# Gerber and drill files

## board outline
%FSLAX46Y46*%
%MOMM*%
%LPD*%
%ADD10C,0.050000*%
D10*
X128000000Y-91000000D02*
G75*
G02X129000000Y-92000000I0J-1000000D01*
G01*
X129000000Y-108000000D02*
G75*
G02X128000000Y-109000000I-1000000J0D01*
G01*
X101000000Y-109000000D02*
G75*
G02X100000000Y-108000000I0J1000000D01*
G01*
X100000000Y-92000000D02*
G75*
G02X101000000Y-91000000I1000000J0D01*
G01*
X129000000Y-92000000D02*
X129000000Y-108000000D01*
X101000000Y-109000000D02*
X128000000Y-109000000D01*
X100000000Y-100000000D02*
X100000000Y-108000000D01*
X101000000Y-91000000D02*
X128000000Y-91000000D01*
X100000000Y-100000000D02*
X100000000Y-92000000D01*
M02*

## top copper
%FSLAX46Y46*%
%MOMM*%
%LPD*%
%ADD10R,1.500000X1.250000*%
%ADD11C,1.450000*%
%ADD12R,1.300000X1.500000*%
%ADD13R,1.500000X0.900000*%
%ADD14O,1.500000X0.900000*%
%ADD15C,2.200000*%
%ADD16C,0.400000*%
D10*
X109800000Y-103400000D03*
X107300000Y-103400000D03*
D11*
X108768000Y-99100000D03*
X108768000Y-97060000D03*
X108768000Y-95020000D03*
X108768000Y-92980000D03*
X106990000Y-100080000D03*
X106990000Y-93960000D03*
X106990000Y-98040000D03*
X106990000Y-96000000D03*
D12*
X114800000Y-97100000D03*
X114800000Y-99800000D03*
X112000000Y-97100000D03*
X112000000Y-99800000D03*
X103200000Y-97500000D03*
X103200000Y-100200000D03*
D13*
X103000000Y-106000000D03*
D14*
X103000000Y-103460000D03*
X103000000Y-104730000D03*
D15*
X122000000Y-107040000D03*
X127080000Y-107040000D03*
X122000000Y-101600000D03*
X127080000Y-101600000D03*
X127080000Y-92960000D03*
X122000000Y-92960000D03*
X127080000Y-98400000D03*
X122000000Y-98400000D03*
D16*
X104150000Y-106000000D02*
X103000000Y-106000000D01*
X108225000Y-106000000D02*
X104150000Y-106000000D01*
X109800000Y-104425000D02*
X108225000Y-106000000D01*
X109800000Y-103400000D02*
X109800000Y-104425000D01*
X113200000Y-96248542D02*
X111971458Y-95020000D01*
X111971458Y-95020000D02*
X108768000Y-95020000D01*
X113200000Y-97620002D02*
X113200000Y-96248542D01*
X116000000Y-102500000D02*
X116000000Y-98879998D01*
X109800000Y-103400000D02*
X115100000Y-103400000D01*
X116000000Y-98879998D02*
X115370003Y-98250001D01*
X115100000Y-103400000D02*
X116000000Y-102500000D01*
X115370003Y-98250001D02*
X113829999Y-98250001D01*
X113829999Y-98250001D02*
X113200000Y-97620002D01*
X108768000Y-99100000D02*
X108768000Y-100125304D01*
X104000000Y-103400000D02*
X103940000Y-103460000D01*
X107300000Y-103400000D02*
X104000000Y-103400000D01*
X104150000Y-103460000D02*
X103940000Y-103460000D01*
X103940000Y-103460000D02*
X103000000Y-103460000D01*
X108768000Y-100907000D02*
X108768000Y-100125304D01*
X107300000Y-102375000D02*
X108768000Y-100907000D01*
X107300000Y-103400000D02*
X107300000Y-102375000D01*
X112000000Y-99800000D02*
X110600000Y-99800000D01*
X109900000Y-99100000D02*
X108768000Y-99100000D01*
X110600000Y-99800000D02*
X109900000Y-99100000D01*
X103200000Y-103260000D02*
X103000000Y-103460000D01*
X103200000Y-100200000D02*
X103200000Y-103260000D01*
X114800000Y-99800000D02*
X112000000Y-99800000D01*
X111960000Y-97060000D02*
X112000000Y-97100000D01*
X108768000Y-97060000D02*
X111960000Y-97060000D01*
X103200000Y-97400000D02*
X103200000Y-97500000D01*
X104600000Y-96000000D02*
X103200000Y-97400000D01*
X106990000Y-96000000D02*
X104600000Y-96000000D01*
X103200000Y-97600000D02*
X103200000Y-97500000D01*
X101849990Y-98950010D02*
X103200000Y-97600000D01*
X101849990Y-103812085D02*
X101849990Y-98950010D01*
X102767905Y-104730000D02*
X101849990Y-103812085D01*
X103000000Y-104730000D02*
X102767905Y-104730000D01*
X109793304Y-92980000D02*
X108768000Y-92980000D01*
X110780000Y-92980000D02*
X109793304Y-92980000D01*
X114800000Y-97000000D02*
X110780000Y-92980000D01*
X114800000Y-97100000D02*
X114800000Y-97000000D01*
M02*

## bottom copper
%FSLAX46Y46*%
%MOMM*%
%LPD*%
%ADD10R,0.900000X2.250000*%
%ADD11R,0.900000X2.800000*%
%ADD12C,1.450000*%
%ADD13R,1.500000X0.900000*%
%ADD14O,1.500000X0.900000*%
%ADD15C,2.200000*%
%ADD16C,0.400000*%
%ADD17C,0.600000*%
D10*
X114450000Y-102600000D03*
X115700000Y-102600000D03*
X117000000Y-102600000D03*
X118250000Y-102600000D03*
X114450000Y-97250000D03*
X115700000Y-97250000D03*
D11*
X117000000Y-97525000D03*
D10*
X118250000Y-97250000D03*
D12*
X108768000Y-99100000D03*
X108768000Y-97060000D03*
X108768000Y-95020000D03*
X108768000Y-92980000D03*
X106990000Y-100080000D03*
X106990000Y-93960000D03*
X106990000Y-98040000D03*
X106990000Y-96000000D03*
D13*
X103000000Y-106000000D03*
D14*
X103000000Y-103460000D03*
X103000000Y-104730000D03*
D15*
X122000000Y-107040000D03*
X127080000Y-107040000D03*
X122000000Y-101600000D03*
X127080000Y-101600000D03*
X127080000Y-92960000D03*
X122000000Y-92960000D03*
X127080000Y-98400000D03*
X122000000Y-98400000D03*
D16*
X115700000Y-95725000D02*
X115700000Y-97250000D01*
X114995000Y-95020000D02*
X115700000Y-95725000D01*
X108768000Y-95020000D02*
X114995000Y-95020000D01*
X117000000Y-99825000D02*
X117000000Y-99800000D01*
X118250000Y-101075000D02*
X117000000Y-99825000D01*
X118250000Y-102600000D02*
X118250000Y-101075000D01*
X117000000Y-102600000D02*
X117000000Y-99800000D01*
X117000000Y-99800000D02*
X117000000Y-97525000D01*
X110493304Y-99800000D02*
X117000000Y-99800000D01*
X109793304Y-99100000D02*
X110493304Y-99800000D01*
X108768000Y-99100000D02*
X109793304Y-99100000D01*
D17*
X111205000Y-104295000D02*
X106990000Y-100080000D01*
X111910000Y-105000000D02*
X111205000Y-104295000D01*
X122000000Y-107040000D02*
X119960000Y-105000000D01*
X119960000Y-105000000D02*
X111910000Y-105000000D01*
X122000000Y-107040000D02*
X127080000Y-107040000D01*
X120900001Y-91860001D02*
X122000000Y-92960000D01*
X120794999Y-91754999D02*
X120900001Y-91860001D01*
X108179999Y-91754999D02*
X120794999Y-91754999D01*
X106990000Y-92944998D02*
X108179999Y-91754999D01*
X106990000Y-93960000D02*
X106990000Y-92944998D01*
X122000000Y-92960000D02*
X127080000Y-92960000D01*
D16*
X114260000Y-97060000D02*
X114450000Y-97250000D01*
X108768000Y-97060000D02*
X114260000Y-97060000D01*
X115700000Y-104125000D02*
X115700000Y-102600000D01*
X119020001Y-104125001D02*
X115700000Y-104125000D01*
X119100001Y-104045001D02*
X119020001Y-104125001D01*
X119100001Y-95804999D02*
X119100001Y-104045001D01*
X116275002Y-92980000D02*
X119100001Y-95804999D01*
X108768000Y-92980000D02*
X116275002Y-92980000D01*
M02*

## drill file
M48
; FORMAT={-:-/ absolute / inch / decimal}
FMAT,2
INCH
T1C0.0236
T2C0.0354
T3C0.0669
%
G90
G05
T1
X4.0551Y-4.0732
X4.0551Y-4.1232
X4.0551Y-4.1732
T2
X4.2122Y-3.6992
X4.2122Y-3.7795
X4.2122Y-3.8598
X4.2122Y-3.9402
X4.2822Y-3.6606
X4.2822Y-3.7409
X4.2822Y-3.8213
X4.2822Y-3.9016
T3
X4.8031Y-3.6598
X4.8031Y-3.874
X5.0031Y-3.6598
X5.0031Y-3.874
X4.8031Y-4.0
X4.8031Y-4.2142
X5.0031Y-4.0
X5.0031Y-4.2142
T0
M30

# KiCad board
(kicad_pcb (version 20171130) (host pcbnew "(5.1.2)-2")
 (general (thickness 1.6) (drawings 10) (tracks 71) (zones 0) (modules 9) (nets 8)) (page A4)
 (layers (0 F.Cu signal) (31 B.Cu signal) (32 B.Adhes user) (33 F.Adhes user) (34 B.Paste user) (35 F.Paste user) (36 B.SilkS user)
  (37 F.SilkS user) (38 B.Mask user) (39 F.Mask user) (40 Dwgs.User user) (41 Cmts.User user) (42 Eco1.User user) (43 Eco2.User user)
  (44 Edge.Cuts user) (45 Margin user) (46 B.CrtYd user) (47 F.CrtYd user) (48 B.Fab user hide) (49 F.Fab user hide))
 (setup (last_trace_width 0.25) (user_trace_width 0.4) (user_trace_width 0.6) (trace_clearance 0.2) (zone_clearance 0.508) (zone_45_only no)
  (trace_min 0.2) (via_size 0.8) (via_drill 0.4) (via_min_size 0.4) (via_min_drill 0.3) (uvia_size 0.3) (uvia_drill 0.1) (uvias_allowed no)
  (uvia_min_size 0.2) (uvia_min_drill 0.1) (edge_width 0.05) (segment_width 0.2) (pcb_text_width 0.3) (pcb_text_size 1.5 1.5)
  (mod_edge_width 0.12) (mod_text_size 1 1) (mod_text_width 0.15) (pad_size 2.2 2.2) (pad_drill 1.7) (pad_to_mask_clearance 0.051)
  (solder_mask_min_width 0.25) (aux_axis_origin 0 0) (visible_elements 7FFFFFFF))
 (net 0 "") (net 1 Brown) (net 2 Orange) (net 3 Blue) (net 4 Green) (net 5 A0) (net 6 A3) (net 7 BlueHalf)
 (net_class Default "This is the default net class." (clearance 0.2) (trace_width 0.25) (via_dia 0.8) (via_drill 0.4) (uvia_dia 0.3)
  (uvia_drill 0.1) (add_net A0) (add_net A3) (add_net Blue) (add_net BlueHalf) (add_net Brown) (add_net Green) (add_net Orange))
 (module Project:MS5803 (layer B.Cu) (at 116.35 100 90)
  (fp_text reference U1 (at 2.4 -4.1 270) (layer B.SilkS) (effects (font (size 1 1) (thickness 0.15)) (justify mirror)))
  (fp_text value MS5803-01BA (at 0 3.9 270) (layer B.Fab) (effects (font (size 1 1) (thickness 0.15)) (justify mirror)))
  (pad 8 smd rect (at -2.6 -1.9 90) (size 2.25 0.9) (layers B.Cu B.Paste B.Mask) (solder_mask_margin 0.1))
  (pad 7 smd rect (at -2.6 -0.65 90) (size 2.25 0.9) (layers B.Cu B.Paste B.Mask) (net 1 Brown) (solder_mask_margin 0.1))
  (pad 6 smd rect (at -2.6 0.65 90) (size 2.25 0.9) (layers B.Cu B.Paste B.Mask) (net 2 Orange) (solder_mask_margin 0.1))
  (pad 5 smd rect (at -2.6 1.9 90) (size 2.25 0.9) (layers B.Cu B.Paste B.Mask) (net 2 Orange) (solder_mask_margin 0.1))
  (pad 1 smd rect (at 2.75 -1.9 90) (size 2.25 0.9) (layers B.Cu B.Paste B.Mask) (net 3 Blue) (solder_mask_margin 0.1))
  (pad 2 smd rect (at 2.75 -0.65 90) (size 2.25 0.9) (layers B.Cu B.Paste B.Mask) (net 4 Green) (solder_mask_margin 0.1))
  (pad 3 smd rect (at 2.475 0.65 90) (size 2.8 0.9) (layers B.Cu B.Paste B.Mask) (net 2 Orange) (solder_mask_margin 0.1))
  (pad 4 smd rect (at 2.75 1.9 90) (size 2.25 0.9) (layers B.Cu B.Paste B.Mask) (solder_mask_margin 0.1)))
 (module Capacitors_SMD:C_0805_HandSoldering (layer F.Cu) (at 108.55 103.4)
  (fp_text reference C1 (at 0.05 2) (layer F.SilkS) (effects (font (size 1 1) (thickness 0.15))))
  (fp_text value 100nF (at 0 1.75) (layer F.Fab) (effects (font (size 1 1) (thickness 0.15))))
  (pad 2 smd rect (at 1.25 0) (size 1.5 1.25) (layers F.Cu F.Paste F.Mask) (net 4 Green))
  (pad 1 smd rect (at -1.25 0) (size 1.5 1.25) (layers F.Cu F.Paste F.Mask) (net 2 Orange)))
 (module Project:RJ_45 (layer F.Cu) (at 107 100.09 270)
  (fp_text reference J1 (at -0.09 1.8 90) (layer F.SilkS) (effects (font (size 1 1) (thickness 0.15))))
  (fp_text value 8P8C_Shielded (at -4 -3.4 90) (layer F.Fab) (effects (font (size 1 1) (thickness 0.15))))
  (pad 2 thru_hole circle (at -0.99 -1.768 270) (size 1.45 1.45) (drill 0.9) (layers *.Cu *.Mask) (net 2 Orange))
  (pad 4 thru_hole circle (at -3.03 -1.768 270) (size 1.45 1.45) (drill 0.9) (layers *.Cu *.Mask) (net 3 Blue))
  (pad 6 thru_hole circle (at -5.07 -1.768 270) (size 1.45 1.45) (drill 0.9) (layers *.Cu *.Mask) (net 4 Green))
  (pad 8 thru_hole circle (at -7.11 -1.768 270) (size 1.45 1.45) (drill 0.9) (layers *.Cu *.Mask) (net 1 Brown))
  (pad 1 thru_hole circle (at -0.01 0.01 270) (size 1.45 1.45) (drill 0.9) (layers *.Cu *.Mask) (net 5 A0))
  (pad 7 thru_hole circle (at -6.13 0.01 270) (size 1.45 1.45) (drill 0.9) (layers *.Cu *.Mask) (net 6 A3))
  (pad 3 thru_hole circle (at -2.05 0.01 270) (size 1.45 1.45) (drill 0.9) (layers *.Cu *.Mask))
  (pad 5 thru_hole circle (at -4.09 0.01 270) (size 1.45 1.45) (drill 0.9) (layers *.Cu *.Mask) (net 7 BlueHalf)))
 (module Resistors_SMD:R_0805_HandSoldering (layer F.Cu) (at 114.8 98.45 90)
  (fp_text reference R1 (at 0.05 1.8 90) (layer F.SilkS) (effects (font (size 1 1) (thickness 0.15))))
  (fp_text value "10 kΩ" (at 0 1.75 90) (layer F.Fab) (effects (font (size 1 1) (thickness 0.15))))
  (pad 2 smd rect (at 1.35 0 90) (size 1.5 1.3) (layers F.Cu F.Paste F.Mask) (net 1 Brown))
  (pad 1 smd rect (at -1.35 0 90) (size 1.5 1.3) (layers F.Cu F.Paste F.Mask) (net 2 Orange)))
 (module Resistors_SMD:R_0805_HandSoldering (layer F.Cu) (at 112 98.45 270)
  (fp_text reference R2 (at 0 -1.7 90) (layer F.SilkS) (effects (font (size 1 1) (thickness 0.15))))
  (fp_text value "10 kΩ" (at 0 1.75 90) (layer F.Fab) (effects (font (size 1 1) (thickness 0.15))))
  (pad 1 smd rect (at -1.35 0 270) (size 1.5 1.3) (layers F.Cu F.Paste F.Mask) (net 3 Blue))
  (pad 2 smd rect (at 1.35 0 270) (size 1.5 1.3) (layers F.Cu F.Paste F.Mask) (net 2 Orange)))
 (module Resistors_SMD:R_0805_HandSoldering (layer F.Cu) (at 103.2 98.85 90)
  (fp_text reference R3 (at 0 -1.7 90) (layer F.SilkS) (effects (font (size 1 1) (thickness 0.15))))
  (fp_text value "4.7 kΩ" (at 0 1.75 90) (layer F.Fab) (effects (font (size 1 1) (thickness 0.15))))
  (pad 2 smd rect (at 1.35 0 90) (size 1.5 1.3) (layers F.Cu F.Paste F.Mask) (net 7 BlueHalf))
  (pad 1 smd rect (at -1.35 0 90) (size 1.5 1.3) (layers F.Cu F.Paste F.Mask) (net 2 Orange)))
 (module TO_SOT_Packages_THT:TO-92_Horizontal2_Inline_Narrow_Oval (layer F.Cu) (at 103 106 90)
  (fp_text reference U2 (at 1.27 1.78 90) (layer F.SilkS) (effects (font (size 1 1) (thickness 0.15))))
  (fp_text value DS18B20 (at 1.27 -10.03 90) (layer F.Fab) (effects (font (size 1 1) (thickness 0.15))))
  (pad 1 thru_hole rect (at 0 0 270) (size 0.9 1.5) (drill 0.6) (layers *.Cu *.Mask) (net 4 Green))
  (pad 3 thru_hole oval (at 2.54 0 270) (size 0.9 1.5) (drill 0.6) (layers *.Cu *.Mask) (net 2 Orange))
  (pad 2 thru_hole oval (at 1.27 0 270) (size 0.9 1.5) (drill 0.6) (layers *.Cu *.Mask) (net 7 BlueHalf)))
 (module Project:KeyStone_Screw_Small (layer F.Cu) (at 122.08 104.32 270)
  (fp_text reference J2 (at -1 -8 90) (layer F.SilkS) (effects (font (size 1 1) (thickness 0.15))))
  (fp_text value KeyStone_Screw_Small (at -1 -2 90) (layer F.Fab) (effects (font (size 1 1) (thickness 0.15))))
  (pad 1 thru_hole circle (at 2.72 0.08) (size 2.2 2.2) (drill 1.7) (layers *.Cu *.Mask) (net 5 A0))
  (pad 1 thru_hole circle (at 2.72 -5 270) (size 2.2 2.2) (drill 1.7) (layers *.Cu *.Mask) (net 5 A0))
  (pad 1 thru_hole circle (at -2.72 0.08) (size 2.2 2.2) (drill 1.7) (layers *.Cu *.Mask))
  (pad 1 thru_hole circle (at -2.72 -5 270) (size 2.2 2.2) (drill 1.7) (layers *.Cu *.Mask)))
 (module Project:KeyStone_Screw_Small (layer F.Cu) (at 122.08 95.68 270)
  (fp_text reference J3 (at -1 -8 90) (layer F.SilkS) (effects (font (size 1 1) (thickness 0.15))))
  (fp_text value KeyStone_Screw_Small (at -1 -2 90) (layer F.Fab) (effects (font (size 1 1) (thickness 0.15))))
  (pad 1 thru_hole circle (at -2.72 -5 270) (size 2.2 2.2) (drill 1.7) (layers *.Cu *.Mask) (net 6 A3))
  (pad 1 thru_hole circle (at -2.72 0.08) (size 2.2 2.2) (drill 1.7) (layers *.Cu *.Mask) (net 6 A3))
  (pad 1 thru_hole circle (at 2.72 -5 270) (size 2.2 2.2) (drill 1.7) (layers *.Cu *.Mask))
  (pad 1 thru_hole circle (at 2.72 0.08) (size 2.2 2.2) (drill 1.7) (layers *.Cu *.Mask)))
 (gr_arc (start 128 92) (end 129 92) (angle -90) (layer Edge.Cuts) (width 0.05))
 (gr_arc (start 128 108) (end 128 109) (angle -90) (layer Edge.Cuts) (width 0.05))
 (gr_arc (start 101 108) (end 100 108) (angle -90) (layer Edge.Cuts) (width 0.05))
 (gr_arc (start 101 92) (end 101 91) (angle -90) (layer Edge.Cuts) (width 0.05))
 (gr_line (start 129 92) (end 129 108) (layer Edge.Cuts) (width 0.05))
 (gr_line (start 101 109) (end 128 109) (layer Edge.Cuts) (width 0.05))
 (gr_line (start 100 100) (end 100 108) (layer Edge.Cuts) (width 0.05))
 (gr_line (start 101 91) (end 128 91) (layer Edge.Cuts) (width 0.05))
 (gr_line (start 100 100) (end 100 92) (layer Edge.Cuts) (width 0.05))
 (segment (start 115.7 95.725) (end 115.7 97.25) (width 0.4) (layer B.Cu) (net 4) (status 20))
 (segment (start 114.995 95.02) (end 115.7 95.725) (width 0.4) (layer B.Cu) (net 4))
 (segment (start 108.768 95.02) (end 114.995 95.02) (width 0.4) (layer B.Cu) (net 4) (status 10))
 (segment (start 104.15 106) (end 103 106) (width 0.4) (layer F.Cu) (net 4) (status 20))
 (segment (start 108.225 106) (end 104.15 106) (width 0.4) (layer F.Cu) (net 4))
 (segment (start 109.8 104.425) (end 108.225 106) (width 0.4) (layer F.Cu) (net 4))
 (segment (start 109.8 103.4) (end 109.8 104.425) (width 0.4) (layer F.Cu) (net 4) (status 10))
 (segment (start 113.2 96.248542) (end 111.971458 95.02) (width 0.4) (layer F.Cu) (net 4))
 (segment (start 111.971458 95.02) (end 108.768 95.02) (width 0.4) (layer F.Cu) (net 4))
 (segment (start 113.2 97.620002) (end 113.2 96.248542) (width 0.4) (layer F.Cu) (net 4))
 (segment (start 116 102.5) (end 116 98.879998) (width 0.4) (layer F.Cu) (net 4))
 (segment (start 109.8 103.4) (end 115.1 103.4) (width 0.4) (layer F.Cu) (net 4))
 (segment (start 116 98.879998) (end 115.370003 98.250001) (width 0.4) (layer F.Cu) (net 4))
 (segment (start 115.1 103.4) (end 116 102.5) (width 0.4) (layer F.Cu) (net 4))
 (segment (start 115.370003 98.250001) (end 113.829999 98.250001) (width 0.4) (layer F.Cu) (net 4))
 (segment (start 113.829999 98.250001) (end 113.2 97.620002) (width 0.4) (layer F.Cu) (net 4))
 (segment (start 117 99.825) (end 117 99.8) (width 0.4) (layer B.Cu) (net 2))
 (segment (start 118.25 101.075) (end 117 99.825) (width 0.4) (layer B.Cu) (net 2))
 (segment (start 118.25 102.6) (end 118.25 101.075) (width 0.4) (layer B.Cu) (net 2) (status 10))
 (segment (start 117 102.6) (end 117 99.8) (width 0.4) (layer B.Cu) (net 2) (status 10))
 (segment (start 117 99.8) (end 117 97.525) (width 0.4) (layer B.Cu) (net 2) (status 20))
 (segment (start 110.493304 99.8) (end 117 99.8) (width 0.4) (layer B.Cu) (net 2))
 (segment (start 109.793304 99.1) (end 110.493304 99.8) (width 0.4) (layer B.Cu) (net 2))
 (segment (start 108.768 99.1) (end 109.793304 99.1) (width 0.4) (layer B.Cu) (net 2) (status 10))
 (segment (start 108.768 99.1) (end 108.768 100.125304) (width 0.4) (layer F.Cu) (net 2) (status 10))
 (segment (start 104 103.4) (end 103.94 103.46) (width 0.4) (layer F.Cu) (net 2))
 (segment (start 107.3 103.4) (end 104 103.4) (width 0.4) (layer F.Cu) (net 2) (status 10))
 (segment (start 104.15 103.46) (end 103.94 103.46) (width 0.4) (layer F.Cu) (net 2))
 (segment (start 103.94 103.46) (end 103 103.46) (width 0.4) (layer F.Cu) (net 2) (status 20))
 (segment (start 108.768 100.907) (end 108.768 100.125304) (width 0.4) (layer F.Cu) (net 2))
 (segment (start 107.3 102.375) (end 108.768 100.907) (width 0.4) (layer F.Cu) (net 2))
 (segment (start 107.3 103.4) (end 107.3 102.375) (width 0.4) (layer F.Cu) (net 2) (status 10))
 (segment (start 112 99.8) (end 110.6 99.8) (width 0.4) (layer F.Cu) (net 2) (status 10))
 (segment (start 109.9 99.1) (end 108.768 99.1) (width 0.4) (layer F.Cu) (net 2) (status 20))
 (segment (start 110.6 99.8) (end 109.9 99.1) (width 0.4) (layer F.Cu) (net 2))
 (segment (start 103.2 103.26) (end 103 103.46) (width 0.4) (layer F.Cu) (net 2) (status 30))
 (segment (start 103.2 100.2) (end 103.2 103.26) (width 0.4) (layer F.Cu) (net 2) (status 30))
 (segment (start 114.8 99.8) (end 112 99.8) (width 0.4) (layer F.Cu) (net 2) (status 30))
 (segment (start 111.205 104.295) (end 106.99 100.08) (width 0.6) (layer B.Cu) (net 5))
 (segment (start 111.91 105) (end 111.205 104.295) (width 0.6) (layer B.Cu) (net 5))
 (segment (start 122 107.04) (end 119.96 105) (width 0.6) (layer B.Cu) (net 5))
 (segment (start 119.96 105) (end 111.91 105) (width 0.6) (layer B.Cu) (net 5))
 (segment (start 122 107.04) (end 127.08 107.04) (width 0.6) (layer B.Cu) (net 5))
 (segment (start 120.900001 91.860001) (end 122 92.96) (width 0.6) (layer B.Cu) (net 6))
 (segment (start 120.794999 91.754999) (end 120.900001 91.860001) (width 0.6) (layer B.Cu) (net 6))
 (segment (start 108.179999 91.754999) (end 120.794999 91.754999) (width 0.6) (layer B.Cu) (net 6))
 (segment (start 106.99 92.944998) (end 108.179999 91.754999) (width 0.6) (layer B.Cu) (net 6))
 (segment (start 106.99 93.96) (end 106.99 92.944998) (width 0.6) (layer B.Cu) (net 6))
 (segment (start 122 92.96) (end 127.08 92.96) (width 0.6) (layer B.Cu) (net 6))
 (segment (start 114.26 97.06) (end 114.45 97.25) (width 0.4) (layer B.Cu) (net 3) (status 30))
 (segment (start 108.768 97.06) (end 114.26 97.06) (width 0.4) (layer B.Cu) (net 3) (status 30))
 (segment (start 111.96 97.06) (end 112 97.1) (width 0.4) (layer F.Cu) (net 3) (status 30))
 (segment (start 108.768 97.06) (end 111.96 97.06) (width 0.4) (layer F.Cu) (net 3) (status 30))
 (segment (start 103.2 97.4) (end 103.2 97.5) (width 0.4) (layer F.Cu) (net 7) (status 30))
 (segment (start 104.6 96) (end 103.2 97.4) (width 0.4) (layer F.Cu) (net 7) (status 20))
 (segment (start 106.99 96) (end 104.6 96) (width 0.4) (layer F.Cu) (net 7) (status 10))
 (segment (start 103.2 97.6) (end 103.2 97.5) (width 0.4) (layer F.Cu) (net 7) (status 30))
 (segment (start 101.84999 98.95001) (end 103.2 97.6) (width 0.4) (layer F.Cu) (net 7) (status 20))
 (segment (start 101.84999 103.812085) (end 101.84999 98.95001) (width 0.4) (layer F.Cu) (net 7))
 (segment (start 102.767905 104.73) (end 101.84999 103.812085) (width 0.4) (layer F.Cu) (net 7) (status 10))
 (segment (start 103 104.73) (end 102.767905 104.73) (width 0.4) (layer F.Cu) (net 7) (status 30))
 (segment (start 115.7 104.125) (end 115.7 102.6) (width 0.4) (layer B.Cu) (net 1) (status 20))
 (segment (start 119.020001 104.125001) (end 115.7 104.125) (width 0.4) (layer B.Cu) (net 1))
 (segment (start 119.100001 104.045001) (end 119.020001 104.125001) (width 0.4) (layer B.Cu) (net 1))
 (segment (start 119.100001 95.804999) (end 119.100001 104.045001) (width 0.4) (layer B.Cu) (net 1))
 (segment (start 116.275002 92.98) (end 119.100001 95.804999) (width 0.4) (layer B.Cu) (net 1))
 (segment (start 108.768 92.98) (end 116.275002 92.98) (width 0.4) (layer B.Cu) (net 1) (status 10))
 (segment (start 109.793304 92.98) (end 108.768 92.98) (width 0.4) (layer F.Cu) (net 1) (status 20))
 (segment (start 110.78 92.98) (end 109.793304 92.98) (width 0.4) (layer F.Cu) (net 1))
 (segment (start 114.8 97) (end 110.78 92.98) (width 0.4) (layer F.Cu) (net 1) (status 10))
 (segment (start 114.8 97.1) (end 114.8 97) (width 0.4) (layer F.Cu) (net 1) (status 30)))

